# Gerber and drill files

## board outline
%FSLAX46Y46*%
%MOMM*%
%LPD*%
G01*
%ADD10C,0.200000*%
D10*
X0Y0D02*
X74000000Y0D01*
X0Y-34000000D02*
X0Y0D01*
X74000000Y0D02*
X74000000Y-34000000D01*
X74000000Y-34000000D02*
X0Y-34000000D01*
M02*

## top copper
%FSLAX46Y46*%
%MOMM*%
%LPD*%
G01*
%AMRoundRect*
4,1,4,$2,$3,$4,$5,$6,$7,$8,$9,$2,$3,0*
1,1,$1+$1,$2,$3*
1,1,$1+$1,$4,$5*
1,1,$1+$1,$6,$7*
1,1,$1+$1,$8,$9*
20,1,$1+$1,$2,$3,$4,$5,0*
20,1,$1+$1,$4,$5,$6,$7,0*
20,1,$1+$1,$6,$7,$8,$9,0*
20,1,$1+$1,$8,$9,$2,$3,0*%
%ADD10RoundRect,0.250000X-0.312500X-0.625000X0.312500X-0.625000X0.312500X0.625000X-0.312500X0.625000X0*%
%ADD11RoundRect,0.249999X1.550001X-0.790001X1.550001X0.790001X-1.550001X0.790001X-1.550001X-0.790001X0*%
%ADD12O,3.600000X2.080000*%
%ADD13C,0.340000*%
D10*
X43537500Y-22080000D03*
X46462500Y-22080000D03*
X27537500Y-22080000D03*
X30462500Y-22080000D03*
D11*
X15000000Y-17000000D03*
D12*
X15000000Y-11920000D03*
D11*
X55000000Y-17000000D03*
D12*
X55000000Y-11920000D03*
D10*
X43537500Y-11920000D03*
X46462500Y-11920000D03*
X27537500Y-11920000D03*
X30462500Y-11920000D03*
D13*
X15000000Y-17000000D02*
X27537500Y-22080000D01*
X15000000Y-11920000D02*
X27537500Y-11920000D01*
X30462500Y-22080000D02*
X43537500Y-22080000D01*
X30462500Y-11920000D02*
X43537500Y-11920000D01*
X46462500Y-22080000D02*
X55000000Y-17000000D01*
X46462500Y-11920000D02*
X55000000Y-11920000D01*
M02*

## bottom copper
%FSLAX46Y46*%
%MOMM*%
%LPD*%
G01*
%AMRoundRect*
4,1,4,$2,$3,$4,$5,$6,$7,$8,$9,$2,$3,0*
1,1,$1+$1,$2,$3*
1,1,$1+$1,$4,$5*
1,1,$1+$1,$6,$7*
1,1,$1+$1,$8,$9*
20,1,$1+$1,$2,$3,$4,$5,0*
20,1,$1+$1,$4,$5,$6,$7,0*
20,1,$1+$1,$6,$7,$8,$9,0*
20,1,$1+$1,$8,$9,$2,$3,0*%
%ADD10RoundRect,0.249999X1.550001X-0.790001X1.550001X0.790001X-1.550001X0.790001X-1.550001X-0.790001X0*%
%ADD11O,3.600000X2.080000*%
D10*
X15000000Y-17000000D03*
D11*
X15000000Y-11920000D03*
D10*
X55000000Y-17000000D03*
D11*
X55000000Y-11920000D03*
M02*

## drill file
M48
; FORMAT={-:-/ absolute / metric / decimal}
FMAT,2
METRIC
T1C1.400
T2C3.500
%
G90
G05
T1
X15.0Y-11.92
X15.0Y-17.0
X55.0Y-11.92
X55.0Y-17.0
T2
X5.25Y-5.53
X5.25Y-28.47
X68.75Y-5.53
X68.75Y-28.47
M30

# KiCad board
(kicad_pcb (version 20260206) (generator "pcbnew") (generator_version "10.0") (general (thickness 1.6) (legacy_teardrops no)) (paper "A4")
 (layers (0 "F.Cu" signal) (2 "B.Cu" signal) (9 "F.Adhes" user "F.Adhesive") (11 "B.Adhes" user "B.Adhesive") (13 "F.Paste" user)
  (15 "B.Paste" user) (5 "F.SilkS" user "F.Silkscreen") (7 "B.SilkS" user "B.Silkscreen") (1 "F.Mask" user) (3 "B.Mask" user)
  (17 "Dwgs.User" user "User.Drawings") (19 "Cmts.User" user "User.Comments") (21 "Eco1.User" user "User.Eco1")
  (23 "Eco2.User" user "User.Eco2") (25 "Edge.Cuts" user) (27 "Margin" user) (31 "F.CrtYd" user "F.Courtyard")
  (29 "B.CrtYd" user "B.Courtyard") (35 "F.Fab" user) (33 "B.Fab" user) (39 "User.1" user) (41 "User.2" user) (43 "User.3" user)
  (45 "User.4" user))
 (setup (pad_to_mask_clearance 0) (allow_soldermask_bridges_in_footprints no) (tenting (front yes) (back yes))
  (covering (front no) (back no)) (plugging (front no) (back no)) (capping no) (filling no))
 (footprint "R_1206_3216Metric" (layer "F.Cu") (at 45 22.08)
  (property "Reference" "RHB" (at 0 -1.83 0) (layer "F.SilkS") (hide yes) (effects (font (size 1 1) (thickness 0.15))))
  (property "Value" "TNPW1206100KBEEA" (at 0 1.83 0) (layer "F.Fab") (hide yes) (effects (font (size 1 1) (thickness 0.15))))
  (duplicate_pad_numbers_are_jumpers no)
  (pad "1" smd roundrect (at -1.4625 0) (size 1.125 1.75) (layers "F.Cu" "F.Mask" "F.Paste") (roundrect_rratio 0.222222) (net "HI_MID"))
  (pad "2" smd roundrect (at 1.4625 0) (size 1.125 1.75) (layers "F.Cu" "F.Mask" "F.Paste") (roundrect_rratio 0.222222) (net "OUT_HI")))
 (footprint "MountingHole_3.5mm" (layer "F.Cu") (at 68.75 5.53)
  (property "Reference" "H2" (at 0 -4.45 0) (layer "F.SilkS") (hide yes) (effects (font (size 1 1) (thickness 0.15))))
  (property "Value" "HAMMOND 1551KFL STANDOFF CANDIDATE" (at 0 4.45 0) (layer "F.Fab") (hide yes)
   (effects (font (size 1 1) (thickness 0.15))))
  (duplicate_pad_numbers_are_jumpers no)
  (pad "" np_thru_hole circle (at 0 0) (size 3.5 3.5) (drill 3.5) (layers "*.Cu" "*.Mask")))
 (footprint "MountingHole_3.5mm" (layer "F.Cu") (at 5.25 28.47)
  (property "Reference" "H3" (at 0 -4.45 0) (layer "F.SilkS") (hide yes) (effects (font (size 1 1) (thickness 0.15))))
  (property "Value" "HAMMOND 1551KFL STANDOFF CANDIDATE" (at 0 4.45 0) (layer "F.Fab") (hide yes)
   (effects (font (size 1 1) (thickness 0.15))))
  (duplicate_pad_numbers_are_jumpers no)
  (pad "" np_thru_hole circle (at 0 0) (size 3.5 3.5) (drill 3.5) (layers "*.Cu" "*.Mask")))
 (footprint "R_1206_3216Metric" (layer "F.Cu") (at 29 22.08)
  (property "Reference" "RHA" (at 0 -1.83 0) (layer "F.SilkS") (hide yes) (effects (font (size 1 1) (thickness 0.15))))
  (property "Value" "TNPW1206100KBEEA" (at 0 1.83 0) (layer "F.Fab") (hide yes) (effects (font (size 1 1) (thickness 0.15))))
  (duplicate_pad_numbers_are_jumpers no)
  (pad "1" smd roundrect (at -1.4625 0) (size 1.125 1.75) (layers "F.Cu" "F.Mask" "F.Paste") (roundrect_rratio 0.222222) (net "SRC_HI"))
  (pad "2" smd roundrect (at 1.4625 0) (size 1.125 1.75) (layers "F.Cu" "F.Mask" "F.Paste") (roundrect_rratio 0.222222) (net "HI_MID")))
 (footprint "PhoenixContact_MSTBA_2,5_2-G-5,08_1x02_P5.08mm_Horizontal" (layer "F.Cu") (at 15 17 90)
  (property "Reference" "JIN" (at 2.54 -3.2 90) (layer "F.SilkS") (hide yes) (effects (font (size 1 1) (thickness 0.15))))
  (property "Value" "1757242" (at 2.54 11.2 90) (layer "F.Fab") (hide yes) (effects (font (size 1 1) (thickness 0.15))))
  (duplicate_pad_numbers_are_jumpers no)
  (pad "1" thru_hole roundrect (at 0 0 90) (size 2.08 3.6) (drill 1.4) (layers "*.Cu" "*.Mask") (remove_unused_layers no)
   (roundrect_rratio 0.120192) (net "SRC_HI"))
  (pad "2" thru_hole oval (at 5.08 0 90) (size 2.08 3.6) (drill 1.4) (layers "*.Cu" "*.Mask") (remove_unused_layers no) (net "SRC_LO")))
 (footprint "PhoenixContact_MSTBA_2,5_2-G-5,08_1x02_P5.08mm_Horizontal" (layer "F.Cu") (at 55 17 90)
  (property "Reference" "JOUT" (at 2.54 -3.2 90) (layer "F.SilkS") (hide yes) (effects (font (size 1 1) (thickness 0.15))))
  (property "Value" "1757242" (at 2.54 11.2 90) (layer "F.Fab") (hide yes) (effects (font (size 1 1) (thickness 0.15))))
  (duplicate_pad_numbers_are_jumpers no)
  (pad "1" thru_hole roundrect (at 0 0 90) (size 2.08 3.6) (drill 1.4) (layers "*.Cu" "*.Mask") (remove_unused_layers no)
   (roundrect_rratio 0.120192) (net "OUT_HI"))
  (pad "2" thru_hole oval (at 5.08 0 90) (size 2.08 3.6) (drill 1.4) (layers "*.Cu" "*.Mask") (remove_unused_layers no) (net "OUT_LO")))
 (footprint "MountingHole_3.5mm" (layer "F.Cu") (at 5.25 5.53)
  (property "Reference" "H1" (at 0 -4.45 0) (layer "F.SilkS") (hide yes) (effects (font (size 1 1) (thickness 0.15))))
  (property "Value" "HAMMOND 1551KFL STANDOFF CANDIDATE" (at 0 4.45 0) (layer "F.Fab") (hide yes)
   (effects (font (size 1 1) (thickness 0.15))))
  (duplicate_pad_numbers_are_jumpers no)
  (pad "" np_thru_hole circle (at 0 0) (size 3.5 3.5) (drill 3.5) (layers "*.Cu" "*.Mask")))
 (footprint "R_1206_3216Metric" (layer "F.Cu") (at 45 11.92)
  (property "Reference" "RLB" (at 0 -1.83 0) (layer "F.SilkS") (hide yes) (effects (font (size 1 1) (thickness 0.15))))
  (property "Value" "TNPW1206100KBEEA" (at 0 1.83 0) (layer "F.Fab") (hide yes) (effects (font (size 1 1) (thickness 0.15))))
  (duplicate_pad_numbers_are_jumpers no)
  (pad "1" smd roundrect (at -1.4625 0) (size 1.125 1.75) (layers "F.Cu" "F.Mask" "F.Paste") (roundrect_rratio 0.222222) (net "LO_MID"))
  (pad "2" smd roundrect (at 1.4625 0) (size 1.125 1.75) (layers "F.Cu" "F.Mask" "F.Paste") (roundrect_rratio 0.222222) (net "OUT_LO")))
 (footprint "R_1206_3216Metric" (layer "F.Cu") (at 29 11.92)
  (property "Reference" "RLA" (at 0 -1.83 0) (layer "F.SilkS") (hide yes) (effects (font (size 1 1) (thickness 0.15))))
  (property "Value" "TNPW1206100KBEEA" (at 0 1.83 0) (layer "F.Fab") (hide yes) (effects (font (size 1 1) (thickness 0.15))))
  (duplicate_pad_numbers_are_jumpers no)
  (pad "1" smd roundrect (at -1.4625 0) (size 1.125 1.75) (layers "F.Cu" "F.Mask" "F.Paste") (roundrect_rratio 0.222222) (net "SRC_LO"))
  (pad "2" smd roundrect (at 1.4625 0) (size 1.125 1.75) (layers "F.Cu" "F.Mask" "F.Paste") (roundrect_rratio 0.222222) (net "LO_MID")))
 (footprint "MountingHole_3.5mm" (layer "F.Cu") (at 68.75 28.47)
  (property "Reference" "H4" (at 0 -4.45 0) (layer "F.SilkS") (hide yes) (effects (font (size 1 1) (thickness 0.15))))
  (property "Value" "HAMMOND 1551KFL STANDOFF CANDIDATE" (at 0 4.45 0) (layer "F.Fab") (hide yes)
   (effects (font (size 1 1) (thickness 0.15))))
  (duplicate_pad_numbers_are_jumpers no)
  (pad "" np_thru_hole circle (at 0 0) (size 3.5 3.5) (drill 3.5) (layers "*.Cu" "*.Mask")))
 (gr_line (start 0 0) (end 74 0) (stroke (width 0.2) (type default)) (layer "Edge.Cuts"))
 (gr_line (start 0 34) (end 0 0) (stroke (width 0.2) (type default)) (layer "Edge.Cuts"))
 (gr_line (start 74 0) (end 74 34) (stroke (width 0.2) (type default)) (layer "Edge.Cuts"))
 (gr_line (start 74 34) (end 0 34) (stroke (width 0.2) (type default)) (layer "Edge.Cuts"))
 (segment (start 15 17) (end 27.5375 22.08) (width 0.34) (layer "F.Cu") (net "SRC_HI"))
 (segment (start 15 11.92) (end 27.5375 11.92) (width 0.34) (layer "F.Cu") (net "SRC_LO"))
 (segment (start 30.4625 22.08) (end 43.5375 22.08) (width 0.34) (layer "F.Cu") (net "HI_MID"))
 (segment (start 30.4625 11.92) (end 43.5375 11.92) (width 0.34) (layer "F.Cu") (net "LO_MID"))
 (segment (start 46.4625 22.08) (end 55 17) (width 0.34) (layer "F.Cu") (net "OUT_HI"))
 (segment (start 46.4625 11.92) (end 55 11.92) (width 0.34) (layer "F.Cu") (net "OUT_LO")))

